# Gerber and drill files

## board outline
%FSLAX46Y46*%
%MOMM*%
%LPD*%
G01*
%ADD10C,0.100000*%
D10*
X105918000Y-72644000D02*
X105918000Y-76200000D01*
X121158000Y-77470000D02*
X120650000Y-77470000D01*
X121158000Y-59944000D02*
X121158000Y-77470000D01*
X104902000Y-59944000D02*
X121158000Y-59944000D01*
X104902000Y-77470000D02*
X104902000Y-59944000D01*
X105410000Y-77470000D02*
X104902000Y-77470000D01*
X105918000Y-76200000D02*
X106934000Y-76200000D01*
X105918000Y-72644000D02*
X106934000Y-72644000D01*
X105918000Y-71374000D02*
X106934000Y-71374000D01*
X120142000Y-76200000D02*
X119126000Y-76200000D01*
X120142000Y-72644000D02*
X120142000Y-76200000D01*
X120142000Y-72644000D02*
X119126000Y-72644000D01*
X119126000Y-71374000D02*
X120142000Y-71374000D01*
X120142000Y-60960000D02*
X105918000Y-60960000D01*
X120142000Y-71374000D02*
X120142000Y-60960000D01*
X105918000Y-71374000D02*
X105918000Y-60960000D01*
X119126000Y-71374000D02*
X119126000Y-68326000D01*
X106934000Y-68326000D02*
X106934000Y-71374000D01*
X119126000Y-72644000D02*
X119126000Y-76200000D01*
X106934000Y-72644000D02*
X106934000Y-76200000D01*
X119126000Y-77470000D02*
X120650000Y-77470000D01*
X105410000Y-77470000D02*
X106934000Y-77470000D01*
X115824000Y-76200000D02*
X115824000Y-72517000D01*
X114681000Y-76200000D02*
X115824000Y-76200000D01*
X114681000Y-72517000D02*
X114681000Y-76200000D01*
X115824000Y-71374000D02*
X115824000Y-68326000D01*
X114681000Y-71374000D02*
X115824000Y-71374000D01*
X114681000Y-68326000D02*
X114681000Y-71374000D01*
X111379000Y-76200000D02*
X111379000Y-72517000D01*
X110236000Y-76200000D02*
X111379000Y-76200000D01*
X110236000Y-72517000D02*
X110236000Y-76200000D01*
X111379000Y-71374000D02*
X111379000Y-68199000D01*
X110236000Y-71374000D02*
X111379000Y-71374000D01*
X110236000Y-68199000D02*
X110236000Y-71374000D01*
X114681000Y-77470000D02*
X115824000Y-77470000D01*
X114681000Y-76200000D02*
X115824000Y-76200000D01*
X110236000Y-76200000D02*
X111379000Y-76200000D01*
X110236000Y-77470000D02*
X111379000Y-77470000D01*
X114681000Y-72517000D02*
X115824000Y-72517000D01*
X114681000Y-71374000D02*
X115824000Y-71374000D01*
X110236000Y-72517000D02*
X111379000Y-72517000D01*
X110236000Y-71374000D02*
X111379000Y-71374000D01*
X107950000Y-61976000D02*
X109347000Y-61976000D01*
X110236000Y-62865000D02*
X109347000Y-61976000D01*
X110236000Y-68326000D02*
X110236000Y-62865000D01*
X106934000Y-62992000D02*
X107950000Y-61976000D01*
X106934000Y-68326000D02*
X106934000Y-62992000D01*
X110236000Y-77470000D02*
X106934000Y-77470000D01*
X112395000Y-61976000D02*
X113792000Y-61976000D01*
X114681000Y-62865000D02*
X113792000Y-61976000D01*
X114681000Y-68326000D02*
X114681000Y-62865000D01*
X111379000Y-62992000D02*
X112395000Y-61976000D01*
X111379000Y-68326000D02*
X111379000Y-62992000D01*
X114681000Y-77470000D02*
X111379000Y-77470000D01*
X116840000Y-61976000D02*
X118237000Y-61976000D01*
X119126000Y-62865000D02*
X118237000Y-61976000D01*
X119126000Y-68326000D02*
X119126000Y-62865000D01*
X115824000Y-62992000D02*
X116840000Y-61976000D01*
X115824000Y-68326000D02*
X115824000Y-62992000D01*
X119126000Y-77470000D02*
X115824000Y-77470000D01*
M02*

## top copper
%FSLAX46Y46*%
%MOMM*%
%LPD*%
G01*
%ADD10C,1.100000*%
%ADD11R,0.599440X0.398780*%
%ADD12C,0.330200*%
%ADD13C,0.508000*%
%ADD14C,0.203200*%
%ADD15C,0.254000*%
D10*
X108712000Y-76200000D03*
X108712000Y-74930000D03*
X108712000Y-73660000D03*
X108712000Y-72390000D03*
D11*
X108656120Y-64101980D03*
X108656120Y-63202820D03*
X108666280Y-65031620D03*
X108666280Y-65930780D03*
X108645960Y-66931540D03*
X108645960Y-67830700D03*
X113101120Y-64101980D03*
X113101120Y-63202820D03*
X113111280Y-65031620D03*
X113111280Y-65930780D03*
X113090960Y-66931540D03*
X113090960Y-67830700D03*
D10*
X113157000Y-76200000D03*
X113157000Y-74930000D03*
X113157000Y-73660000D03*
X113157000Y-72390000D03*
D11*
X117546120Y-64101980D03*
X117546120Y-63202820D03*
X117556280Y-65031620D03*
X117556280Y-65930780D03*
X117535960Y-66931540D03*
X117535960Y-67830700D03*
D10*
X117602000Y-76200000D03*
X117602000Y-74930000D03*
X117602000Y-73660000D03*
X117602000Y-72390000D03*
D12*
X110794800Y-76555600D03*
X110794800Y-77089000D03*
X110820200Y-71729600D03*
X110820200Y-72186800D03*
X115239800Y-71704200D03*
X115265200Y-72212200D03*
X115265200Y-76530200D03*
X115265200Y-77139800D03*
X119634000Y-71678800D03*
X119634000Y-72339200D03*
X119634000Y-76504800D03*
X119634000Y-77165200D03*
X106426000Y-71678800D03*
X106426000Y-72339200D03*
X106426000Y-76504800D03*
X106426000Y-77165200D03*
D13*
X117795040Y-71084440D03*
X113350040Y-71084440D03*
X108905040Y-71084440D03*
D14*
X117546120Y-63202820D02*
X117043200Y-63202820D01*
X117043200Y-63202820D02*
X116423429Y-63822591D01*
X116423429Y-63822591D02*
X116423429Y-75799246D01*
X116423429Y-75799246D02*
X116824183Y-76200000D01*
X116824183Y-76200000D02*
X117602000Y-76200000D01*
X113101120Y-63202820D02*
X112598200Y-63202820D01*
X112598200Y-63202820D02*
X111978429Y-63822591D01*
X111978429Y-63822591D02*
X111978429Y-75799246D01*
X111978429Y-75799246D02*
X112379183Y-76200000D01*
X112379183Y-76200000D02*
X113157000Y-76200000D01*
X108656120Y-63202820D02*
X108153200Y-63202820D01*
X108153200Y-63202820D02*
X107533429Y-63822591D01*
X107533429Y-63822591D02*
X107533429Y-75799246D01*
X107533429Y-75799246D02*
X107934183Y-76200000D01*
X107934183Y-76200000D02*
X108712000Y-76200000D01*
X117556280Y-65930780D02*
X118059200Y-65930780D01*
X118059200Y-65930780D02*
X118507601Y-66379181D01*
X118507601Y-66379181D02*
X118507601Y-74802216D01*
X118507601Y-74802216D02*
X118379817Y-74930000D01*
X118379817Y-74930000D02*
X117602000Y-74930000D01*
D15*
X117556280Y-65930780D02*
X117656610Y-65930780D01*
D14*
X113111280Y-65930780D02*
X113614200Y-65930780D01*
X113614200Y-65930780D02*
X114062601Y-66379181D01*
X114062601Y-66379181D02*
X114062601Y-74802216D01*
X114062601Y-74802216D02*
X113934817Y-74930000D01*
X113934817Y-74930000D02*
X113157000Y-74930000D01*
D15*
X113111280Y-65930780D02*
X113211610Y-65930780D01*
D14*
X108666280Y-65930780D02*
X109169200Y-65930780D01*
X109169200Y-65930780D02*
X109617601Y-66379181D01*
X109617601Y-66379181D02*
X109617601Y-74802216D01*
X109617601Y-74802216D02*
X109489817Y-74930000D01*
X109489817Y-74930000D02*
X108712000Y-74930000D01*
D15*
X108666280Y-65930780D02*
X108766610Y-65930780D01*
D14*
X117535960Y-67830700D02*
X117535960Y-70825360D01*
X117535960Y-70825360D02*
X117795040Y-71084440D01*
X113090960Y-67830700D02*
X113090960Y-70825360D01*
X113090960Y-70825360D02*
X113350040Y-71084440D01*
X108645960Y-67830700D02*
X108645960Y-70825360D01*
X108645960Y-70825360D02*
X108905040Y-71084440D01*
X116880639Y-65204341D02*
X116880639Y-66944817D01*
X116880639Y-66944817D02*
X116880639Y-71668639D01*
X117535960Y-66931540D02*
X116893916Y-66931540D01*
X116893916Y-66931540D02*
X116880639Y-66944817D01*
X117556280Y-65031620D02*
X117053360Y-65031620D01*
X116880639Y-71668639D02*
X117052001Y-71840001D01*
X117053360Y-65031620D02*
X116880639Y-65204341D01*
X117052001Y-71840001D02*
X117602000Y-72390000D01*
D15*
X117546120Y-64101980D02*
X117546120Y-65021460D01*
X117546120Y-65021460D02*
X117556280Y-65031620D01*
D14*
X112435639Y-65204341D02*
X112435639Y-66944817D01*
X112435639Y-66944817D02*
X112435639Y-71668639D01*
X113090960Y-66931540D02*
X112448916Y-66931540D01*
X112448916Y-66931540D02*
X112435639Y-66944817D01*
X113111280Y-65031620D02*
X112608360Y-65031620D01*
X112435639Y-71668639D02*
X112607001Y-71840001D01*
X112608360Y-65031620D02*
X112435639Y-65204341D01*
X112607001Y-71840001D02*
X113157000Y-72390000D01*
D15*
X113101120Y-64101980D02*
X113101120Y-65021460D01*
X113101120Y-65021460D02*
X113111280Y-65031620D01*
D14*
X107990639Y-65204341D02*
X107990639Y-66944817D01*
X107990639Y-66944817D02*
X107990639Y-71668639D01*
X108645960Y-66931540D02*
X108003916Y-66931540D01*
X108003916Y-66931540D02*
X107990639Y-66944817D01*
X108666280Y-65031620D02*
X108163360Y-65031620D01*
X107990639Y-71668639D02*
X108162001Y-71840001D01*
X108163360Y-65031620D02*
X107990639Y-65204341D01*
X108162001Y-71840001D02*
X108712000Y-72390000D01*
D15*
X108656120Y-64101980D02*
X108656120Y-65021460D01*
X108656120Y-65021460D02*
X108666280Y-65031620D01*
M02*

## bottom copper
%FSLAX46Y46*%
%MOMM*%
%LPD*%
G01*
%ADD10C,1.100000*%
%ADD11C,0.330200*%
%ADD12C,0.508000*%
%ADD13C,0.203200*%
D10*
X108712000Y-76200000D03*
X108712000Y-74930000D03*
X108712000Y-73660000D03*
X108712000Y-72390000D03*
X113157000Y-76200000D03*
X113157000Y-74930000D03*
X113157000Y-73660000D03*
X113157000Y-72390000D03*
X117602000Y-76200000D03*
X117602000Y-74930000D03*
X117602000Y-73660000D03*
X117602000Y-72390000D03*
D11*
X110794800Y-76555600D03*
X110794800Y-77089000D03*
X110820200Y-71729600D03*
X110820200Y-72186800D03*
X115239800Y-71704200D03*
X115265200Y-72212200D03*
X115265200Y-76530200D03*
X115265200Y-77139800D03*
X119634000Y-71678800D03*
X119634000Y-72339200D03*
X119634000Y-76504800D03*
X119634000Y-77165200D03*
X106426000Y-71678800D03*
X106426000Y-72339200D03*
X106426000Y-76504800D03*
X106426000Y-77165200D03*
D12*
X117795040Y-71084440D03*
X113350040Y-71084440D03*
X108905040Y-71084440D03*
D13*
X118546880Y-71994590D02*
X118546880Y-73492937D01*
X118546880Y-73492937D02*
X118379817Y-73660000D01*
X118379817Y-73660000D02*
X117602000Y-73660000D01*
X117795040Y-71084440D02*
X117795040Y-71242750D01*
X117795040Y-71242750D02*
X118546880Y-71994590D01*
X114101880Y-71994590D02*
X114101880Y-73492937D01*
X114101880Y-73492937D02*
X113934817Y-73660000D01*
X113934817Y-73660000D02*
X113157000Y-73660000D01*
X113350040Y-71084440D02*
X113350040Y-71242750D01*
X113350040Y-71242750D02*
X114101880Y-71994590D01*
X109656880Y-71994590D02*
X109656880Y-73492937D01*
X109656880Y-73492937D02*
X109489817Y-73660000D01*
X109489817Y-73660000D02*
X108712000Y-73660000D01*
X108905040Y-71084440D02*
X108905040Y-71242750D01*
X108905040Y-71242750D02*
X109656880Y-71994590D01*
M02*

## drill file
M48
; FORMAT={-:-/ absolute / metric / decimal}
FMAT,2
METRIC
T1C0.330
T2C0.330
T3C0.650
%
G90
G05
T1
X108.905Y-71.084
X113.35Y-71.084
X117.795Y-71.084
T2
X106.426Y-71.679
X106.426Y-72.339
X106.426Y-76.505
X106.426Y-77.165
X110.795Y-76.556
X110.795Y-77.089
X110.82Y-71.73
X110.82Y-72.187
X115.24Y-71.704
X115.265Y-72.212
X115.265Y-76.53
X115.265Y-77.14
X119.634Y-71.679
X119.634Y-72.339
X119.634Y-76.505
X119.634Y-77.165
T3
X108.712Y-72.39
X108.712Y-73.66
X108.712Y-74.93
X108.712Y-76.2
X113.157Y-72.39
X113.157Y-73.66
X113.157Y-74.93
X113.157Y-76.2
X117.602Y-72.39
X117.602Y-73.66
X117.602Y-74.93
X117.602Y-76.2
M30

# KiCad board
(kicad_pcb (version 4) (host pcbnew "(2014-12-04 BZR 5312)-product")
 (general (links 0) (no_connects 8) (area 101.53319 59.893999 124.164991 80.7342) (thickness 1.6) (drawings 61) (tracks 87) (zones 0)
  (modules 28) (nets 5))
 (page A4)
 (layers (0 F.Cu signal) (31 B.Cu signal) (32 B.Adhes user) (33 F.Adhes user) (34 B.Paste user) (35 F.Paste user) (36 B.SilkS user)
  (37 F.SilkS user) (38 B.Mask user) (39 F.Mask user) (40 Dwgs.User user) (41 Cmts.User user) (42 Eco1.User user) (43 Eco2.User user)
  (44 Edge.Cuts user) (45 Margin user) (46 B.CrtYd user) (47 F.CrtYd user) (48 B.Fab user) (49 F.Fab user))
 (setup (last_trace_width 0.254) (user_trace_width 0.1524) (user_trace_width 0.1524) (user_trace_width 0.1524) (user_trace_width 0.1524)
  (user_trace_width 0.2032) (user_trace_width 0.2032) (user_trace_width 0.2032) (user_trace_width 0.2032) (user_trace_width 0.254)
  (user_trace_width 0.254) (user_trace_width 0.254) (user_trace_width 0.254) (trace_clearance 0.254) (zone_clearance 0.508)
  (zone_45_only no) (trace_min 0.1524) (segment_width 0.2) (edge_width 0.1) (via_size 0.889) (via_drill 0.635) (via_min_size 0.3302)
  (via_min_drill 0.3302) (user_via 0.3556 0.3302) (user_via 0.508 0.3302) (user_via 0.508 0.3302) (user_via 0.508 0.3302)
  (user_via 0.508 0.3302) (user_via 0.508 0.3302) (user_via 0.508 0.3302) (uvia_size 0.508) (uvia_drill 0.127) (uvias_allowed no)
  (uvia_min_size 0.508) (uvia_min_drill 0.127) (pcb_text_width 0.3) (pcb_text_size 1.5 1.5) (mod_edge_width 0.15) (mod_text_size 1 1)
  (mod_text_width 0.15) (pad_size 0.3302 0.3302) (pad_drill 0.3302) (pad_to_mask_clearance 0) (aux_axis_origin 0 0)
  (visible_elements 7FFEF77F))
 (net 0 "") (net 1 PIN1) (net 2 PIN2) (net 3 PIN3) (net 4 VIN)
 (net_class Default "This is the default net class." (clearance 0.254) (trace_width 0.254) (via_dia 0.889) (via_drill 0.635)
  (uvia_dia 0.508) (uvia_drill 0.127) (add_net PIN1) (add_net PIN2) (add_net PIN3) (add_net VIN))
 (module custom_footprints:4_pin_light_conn (layer F.Cu) (at 112.522 76.2 90)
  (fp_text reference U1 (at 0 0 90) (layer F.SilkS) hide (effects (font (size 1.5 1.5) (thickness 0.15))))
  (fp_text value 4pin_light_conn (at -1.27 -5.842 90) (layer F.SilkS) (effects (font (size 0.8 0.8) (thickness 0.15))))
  (pad 1 thru_hole circle (at 0 -3.81 90) (size 1.1 1.1) (drill 0.65) (layers *.Cu *.Mask F.SilkS) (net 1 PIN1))
  (pad 2 thru_hole circle (at 1.27 -3.81 90) (size 1.1 1.1) (drill 0.65) (layers *.Cu *.Mask F.SilkS) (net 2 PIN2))
  (pad 3 thru_hole circle (at 2.54 -3.81 90) (size 1.1 1.1) (drill 0.65) (layers *.Cu *.Mask F.SilkS) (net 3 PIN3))
  (pad 4 thru_hole circle (at 3.81 -3.81 90) (size 1.1 1.1) (drill 0.65) (layers *.Cu *.Mask F.SilkS) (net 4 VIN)))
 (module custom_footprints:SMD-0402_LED (layer F.Cu) (at 108.65612 63.6524 90)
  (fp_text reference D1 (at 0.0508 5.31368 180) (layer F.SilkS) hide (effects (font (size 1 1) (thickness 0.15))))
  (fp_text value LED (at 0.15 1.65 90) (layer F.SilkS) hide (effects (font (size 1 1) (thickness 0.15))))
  (pad 1 smd rect (at -0.44958 0 90) (size 0.39878 0.59944) (layers F.Cu F.Paste F.Mask) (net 4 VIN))
  (pad 2 smd rect (at 0.44958 0 90) (size 0.39878 0.59944) (layers F.Cu F.Paste F.Mask) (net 1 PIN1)))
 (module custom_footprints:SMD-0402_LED (layer F.Cu) (at 108.66628 65.4812 270)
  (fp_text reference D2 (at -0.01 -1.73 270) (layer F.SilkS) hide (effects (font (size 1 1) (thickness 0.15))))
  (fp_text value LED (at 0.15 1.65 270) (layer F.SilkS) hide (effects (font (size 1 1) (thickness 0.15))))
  (pad 1 smd rect (at -0.44958 0 270) (size 0.39878 0.59944) (layers F.Cu F.Paste F.Mask) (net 4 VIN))
  (pad 2 smd rect (at 0.44958 0 270) (size 0.39878 0.59944) (layers F.Cu F.Paste F.Mask) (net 2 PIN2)))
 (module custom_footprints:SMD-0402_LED (layer F.Cu) (at 108.64596 67.38112 270)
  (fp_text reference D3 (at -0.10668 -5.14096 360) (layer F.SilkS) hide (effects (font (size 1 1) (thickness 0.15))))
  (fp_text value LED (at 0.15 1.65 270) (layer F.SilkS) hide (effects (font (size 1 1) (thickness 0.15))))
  (pad 1 smd rect (at -0.44958 0 270) (size 0.39878 0.59944) (layers F.Cu F.Paste F.Mask) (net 4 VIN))
  (pad 2 smd rect (at 0.44958 0 270) (size 0.39878 0.59944) (layers F.Cu F.Paste F.Mask) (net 3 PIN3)))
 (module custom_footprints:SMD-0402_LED (layer F.Cu) (at 113.10112 63.6524 90)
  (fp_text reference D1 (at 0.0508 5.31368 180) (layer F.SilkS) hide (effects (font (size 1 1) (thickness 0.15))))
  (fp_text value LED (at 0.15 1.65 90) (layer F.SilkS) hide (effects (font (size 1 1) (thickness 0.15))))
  (pad 1 smd rect (at -0.44958 0 90) (size 0.39878 0.59944) (layers F.Cu F.Paste F.Mask) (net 4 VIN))
  (pad 2 smd rect (at 0.44958 0 90) (size 0.39878 0.59944) (layers F.Cu F.Paste F.Mask) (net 1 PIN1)))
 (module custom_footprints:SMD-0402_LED (layer F.Cu) (at 113.11128 65.4812 270)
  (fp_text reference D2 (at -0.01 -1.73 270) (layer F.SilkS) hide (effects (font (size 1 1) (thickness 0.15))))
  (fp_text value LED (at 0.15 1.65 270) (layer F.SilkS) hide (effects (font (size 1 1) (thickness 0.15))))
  (pad 1 smd rect (at -0.44958 0 270) (size 0.39878 0.59944) (layers F.Cu F.Paste F.Mask) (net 4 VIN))
  (pad 2 smd rect (at 0.44958 0 270) (size 0.39878 0.59944) (layers F.Cu F.Paste F.Mask) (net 2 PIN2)))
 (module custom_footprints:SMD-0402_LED (layer F.Cu) (at 113.09096 67.38112 270)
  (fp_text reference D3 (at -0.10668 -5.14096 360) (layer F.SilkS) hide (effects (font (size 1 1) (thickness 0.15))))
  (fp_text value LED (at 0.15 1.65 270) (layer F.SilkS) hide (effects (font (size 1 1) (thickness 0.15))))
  (pad 1 smd rect (at -0.44958 0 270) (size 0.39878 0.59944) (layers F.Cu F.Paste F.Mask) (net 4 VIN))
  (pad 2 smd rect (at 0.44958 0 270) (size 0.39878 0.59944) (layers F.Cu F.Paste F.Mask) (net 3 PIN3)))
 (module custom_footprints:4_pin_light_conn (layer F.Cu) (at 116.967 76.2 90)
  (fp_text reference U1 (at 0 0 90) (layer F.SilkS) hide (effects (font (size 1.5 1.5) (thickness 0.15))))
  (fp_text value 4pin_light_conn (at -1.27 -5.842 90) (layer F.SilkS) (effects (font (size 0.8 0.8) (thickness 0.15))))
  (pad 1 thru_hole circle (at 0 -3.81 90) (size 1.1 1.1) (drill 0.65) (layers *.Cu *.Mask F.SilkS) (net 1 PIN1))
  (pad 2 thru_hole circle (at 1.27 -3.81 90) (size 1.1 1.1) (drill 0.65) (layers *.Cu *.Mask F.SilkS) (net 2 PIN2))
  (pad 3 thru_hole circle (at 2.54 -3.81 90) (size 1.1 1.1) (drill 0.65) (layers *.Cu *.Mask F.SilkS) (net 3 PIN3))
  (pad 4 thru_hole circle (at 3.81 -3.81 90) (size 1.1 1.1) (drill 0.65) (layers *.Cu *.Mask F.SilkS) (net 4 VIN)))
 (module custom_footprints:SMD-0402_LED (layer F.Cu) (at 117.54612 63.6524 90)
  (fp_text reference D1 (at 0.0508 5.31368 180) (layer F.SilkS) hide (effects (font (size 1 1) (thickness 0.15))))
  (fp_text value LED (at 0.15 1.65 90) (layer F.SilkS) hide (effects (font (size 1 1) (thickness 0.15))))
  (pad 1 smd rect (at -0.44958 0 90) (size 0.39878 0.59944) (layers F.Cu F.Paste F.Mask) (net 4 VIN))
  (pad 2 smd rect (at 0.44958 0 90) (size 0.39878 0.59944) (layers F.Cu F.Paste F.Mask) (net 1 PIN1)))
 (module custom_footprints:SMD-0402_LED (layer F.Cu) (at 117.55628 65.4812 270)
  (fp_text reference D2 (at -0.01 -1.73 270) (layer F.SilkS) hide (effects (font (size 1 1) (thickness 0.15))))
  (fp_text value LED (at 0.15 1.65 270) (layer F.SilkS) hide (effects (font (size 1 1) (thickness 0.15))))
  (pad 1 smd rect (at -0.44958 0 270) (size 0.39878 0.59944) (layers F.Cu F.Paste F.Mask) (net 4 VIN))
  (pad 2 smd rect (at 0.44958 0 270) (size 0.39878 0.59944) (layers F.Cu F.Paste F.Mask) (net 2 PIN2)))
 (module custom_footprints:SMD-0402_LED (layer F.Cu) (at 117.53596 67.38112 270)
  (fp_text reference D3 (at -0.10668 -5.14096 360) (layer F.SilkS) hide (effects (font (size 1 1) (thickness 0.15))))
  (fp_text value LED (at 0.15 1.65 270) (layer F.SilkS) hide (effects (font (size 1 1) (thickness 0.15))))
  (pad 1 smd rect (at -0.44958 0 270) (size 0.39878 0.59944) (layers F.Cu F.Paste F.Mask) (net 4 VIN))
  (pad 2 smd rect (at 0.44958 0 270) (size 0.39878 0.59944) (layers F.Cu F.Paste F.Mask) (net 3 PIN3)))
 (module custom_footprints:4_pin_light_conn (layer F.Cu) (at 121.412 76.2 90)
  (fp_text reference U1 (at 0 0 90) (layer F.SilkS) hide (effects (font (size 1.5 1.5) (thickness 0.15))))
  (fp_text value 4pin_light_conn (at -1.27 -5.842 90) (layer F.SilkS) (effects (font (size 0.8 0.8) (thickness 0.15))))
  (pad 1 thru_hole circle (at 0 -3.81 90) (size 1.1 1.1) (drill 0.65) (layers *.Cu *.Mask F.SilkS) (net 1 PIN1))
  (pad 2 thru_hole circle (at 1.27 -3.81 90) (size 1.1 1.1) (drill 0.65) (layers *.Cu *.Mask F.SilkS) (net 2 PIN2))
  (pad 3 thru_hole circle (at 2.54 -3.81 90) (size 1.1 1.1) (drill 0.65) (layers *.Cu *.Mask F.SilkS) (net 3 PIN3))
  (pad 4 thru_hole circle (at 3.81 -3.81 90) (size 1.1 1.1) (drill 0.65) (layers *.Cu *.Mask F.SilkS) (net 4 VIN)))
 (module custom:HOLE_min (layer F.Cu) (at 110.7948 76.5556)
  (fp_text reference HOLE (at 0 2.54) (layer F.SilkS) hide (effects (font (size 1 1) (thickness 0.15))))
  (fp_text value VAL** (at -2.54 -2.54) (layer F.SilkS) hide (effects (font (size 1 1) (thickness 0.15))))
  (pad 1 thru_hole circle (at 0 0) (size 0.3302 0.3302) (drill 0.3302) (layers *.Cu *.Mask F.SilkS)))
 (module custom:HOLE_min (layer F.Cu) (at 110.7948 77.089)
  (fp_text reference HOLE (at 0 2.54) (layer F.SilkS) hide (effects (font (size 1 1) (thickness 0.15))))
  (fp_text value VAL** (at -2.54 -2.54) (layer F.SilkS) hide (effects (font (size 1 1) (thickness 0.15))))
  (pad 1 thru_hole circle (at 0 0) (size 0.3302 0.3302) (drill 0.3302) (layers *.Cu *.Mask F.SilkS)))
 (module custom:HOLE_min (layer F.Cu) (at 110.8202 71.7296)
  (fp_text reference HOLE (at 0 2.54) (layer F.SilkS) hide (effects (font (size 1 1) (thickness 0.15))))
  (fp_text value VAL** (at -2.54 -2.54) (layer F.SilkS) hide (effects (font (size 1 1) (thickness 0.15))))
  (pad 1 thru_hole circle (at 0 0) (size 0.3302 0.3302) (drill 0.3302) (layers *.Cu *.Mask F.SilkS)))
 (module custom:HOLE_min (layer F.Cu) (at 110.8202 72.1868)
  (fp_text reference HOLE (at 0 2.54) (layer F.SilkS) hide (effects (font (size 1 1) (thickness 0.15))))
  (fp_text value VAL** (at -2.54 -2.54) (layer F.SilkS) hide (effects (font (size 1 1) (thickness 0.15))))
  (pad 1 thru_hole circle (at 0 0) (size 0.3302 0.3302) (drill 0.3302) (layers *.Cu *.Mask F.SilkS)))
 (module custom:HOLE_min (layer F.Cu) (at 115.2398 71.7042)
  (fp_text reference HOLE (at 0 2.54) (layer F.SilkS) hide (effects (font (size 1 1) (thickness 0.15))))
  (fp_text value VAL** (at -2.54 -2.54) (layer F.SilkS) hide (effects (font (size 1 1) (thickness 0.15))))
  (pad 1 thru_hole circle (at 0 0) (size 0.3302 0.3302) (drill 0.3302) (layers *.Cu *.Mask F.SilkS)))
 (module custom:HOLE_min (layer F.Cu) (at 115.2652 72.2122)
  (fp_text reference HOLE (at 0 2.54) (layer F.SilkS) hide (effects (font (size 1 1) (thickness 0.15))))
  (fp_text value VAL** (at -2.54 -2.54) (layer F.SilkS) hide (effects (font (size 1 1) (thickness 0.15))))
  (pad 1 thru_hole circle (at 0 0) (size 0.3302 0.3302) (drill 0.3302) (layers *.Cu *.Mask F.SilkS)))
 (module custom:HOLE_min (layer F.Cu) (at 115.2652 76.5302)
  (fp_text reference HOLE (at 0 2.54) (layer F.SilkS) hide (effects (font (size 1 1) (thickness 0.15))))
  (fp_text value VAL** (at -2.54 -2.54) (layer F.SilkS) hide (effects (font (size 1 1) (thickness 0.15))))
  (pad 1 thru_hole circle (at 0 0) (size 0.3302 0.3302) (drill 0.3302) (layers *.Cu *.Mask F.SilkS)))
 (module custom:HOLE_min (layer F.Cu) (at 115.2652 77.1398)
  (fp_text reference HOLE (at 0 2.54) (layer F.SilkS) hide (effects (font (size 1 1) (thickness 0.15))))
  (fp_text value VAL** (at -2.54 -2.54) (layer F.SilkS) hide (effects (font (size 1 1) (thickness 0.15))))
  (pad 1 thru_hole circle (at 0 0) (size 0.3302 0.3302) (drill 0.3302) (layers *.Cu *.Mask F.SilkS)))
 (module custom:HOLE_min (layer F.Cu) (at 119.634 71.6788)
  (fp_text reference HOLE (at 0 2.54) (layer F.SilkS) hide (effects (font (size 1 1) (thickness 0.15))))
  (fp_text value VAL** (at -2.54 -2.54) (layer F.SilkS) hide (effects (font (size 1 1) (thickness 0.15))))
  (pad 1 thru_hole circle (at 0 0) (size 0.3302 0.3302) (drill 0.3302) (layers *.Cu *.Mask F.SilkS)))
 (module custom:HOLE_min (layer F.Cu) (at 119.634 72.3392)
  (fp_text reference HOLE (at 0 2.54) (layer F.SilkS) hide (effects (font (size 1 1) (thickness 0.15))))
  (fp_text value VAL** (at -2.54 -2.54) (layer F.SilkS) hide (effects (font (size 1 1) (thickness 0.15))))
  (pad 1 thru_hole circle (at 0 0) (size 0.3302 0.3302) (drill 0.3302) (layers *.Cu *.Mask F.SilkS)))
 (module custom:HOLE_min (layer F.Cu) (at 119.634 76.5048)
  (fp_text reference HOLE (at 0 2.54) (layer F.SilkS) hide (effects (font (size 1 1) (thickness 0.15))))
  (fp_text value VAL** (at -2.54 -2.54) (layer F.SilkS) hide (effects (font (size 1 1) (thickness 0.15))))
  (pad 1 thru_hole circle (at 0 0) (size 0.3302 0.3302) (drill 0.3302) (layers *.Cu *.Mask F.SilkS)))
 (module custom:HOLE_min (layer F.Cu) (at 119.634 77.1652)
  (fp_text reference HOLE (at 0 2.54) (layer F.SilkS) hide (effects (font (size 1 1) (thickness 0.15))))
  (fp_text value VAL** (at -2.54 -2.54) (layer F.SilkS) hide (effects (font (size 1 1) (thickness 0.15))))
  (pad 1 thru_hole circle (at 0 0) (size 0.3302 0.3302) (drill 0.3302) (layers *.Cu *.Mask F.SilkS)))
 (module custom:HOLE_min (layer F.Cu) (at 106.426 71.6788)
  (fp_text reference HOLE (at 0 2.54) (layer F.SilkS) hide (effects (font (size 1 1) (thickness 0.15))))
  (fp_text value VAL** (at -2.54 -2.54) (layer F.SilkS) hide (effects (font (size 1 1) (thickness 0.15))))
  (pad 1 thru_hole circle (at 0 0) (size 0.3302 0.3302) (drill 0.3302) (layers *.Cu *.Mask F.SilkS)))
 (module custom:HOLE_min (layer F.Cu) (at 106.426 72.3392)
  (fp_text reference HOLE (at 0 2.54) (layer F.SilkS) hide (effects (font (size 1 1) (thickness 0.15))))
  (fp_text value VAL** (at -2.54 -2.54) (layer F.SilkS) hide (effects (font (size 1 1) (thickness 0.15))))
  (pad 1 thru_hole circle (at 0 0) (size 0.3302 0.3302) (drill 0.3302) (layers *.Cu *.Mask F.SilkS)))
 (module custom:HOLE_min (layer F.Cu) (at 106.426 76.5048)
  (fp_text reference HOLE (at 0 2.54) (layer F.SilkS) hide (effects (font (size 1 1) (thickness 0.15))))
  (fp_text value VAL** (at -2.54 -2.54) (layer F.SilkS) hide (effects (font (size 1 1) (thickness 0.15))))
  (pad 1 thru_hole circle (at 0 0) (size 0.3302 0.3302) (drill 0.3302) (layers *.Cu *.Mask F.SilkS)))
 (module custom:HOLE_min (layer F.Cu) (at 106.426 77.1652)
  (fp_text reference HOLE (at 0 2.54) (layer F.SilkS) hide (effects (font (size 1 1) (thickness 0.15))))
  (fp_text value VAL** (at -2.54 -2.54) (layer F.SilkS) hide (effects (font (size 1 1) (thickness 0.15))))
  (pad 1 thru_hole circle (at 0 0) (size 0.3302 0.3302) (drill 0.3302) (layers *.Cu *.Mask F.SilkS)))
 (gr_line (start 105.918 72.644) (end 105.918 76.2) (angle 90) (layer Edge.Cuts) (width 0.1))
 (gr_line (start 121.158 77.47) (end 120.65 77.47) (angle 90) (layer Edge.Cuts) (width 0.1))
 (gr_line (start 121.158 59.944) (end 121.158 77.47) (angle 90) (layer Edge.Cuts) (width 0.1))
 (gr_line (start 104.902 59.944) (end 121.158 59.944) (angle 90) (layer Edge.Cuts) (width 0.1))
 (gr_line (start 104.902 77.47) (end 104.902 59.944) (angle 90) (layer Edge.Cuts) (width 0.1))
 (gr_line (start 105.41 77.47) (end 104.902 77.47) (angle 90) (layer Edge.Cuts) (width 0.1))
 (gr_line (start 105.918 76.2) (end 106.934 76.2) (angle 90) (layer Edge.Cuts) (width 0.1))
 (gr_line (start 105.918 72.644) (end 106.934 72.644) (angle 90) (layer Edge.Cuts) (width 0.1))
 (gr_line (start 105.918 71.374) (end 106.934 71.374) (angle 90) (layer Edge.Cuts) (width 0.1))
 (gr_line (start 120.142 76.2) (end 119.126 76.2) (angle 90) (layer Edge.Cuts) (width 0.1))
 (gr_line (start 120.142 72.644) (end 120.142 76.2) (angle 90) (layer Edge.Cuts) (width 0.1))
 (gr_line (start 120.142 72.644) (end 119.126 72.644) (angle 90) (layer Edge.Cuts) (width 0.1))
 (gr_line (start 119.126 71.374) (end 120.142 71.374) (angle 90) (layer Edge.Cuts) (width 0.1))
 (gr_line (start 120.142 60.96) (end 105.918 60.96) (angle 90) (layer Edge.Cuts) (width 0.1))
 (gr_line (start 120.142 71.374) (end 120.142 60.96) (angle 90) (layer Edge.Cuts) (width 0.1))
 (gr_line (start 105.918 71.374) (end 105.918 60.96) (angle 90) (layer Edge.Cuts) (width 0.1))
 (gr_line (start 119.126 71.374) (end 119.126 68.326) (angle 90) (layer Edge.Cuts) (width 0.1))
 (gr_line (start 106.934 68.326) (end 106.934 71.374) (angle 90) (layer Edge.Cuts) (width 0.1))
 (gr_line (start 119.126 72.644) (end 119.126 76.2) (angle 90) (layer Edge.Cuts) (width 0.1))
 (gr_line (start 106.934 72.644) (end 106.934 76.2) (angle 90) (layer Edge.Cuts) (width 0.1))
 (gr_line (start 119.126 77.47) (end 120.65 77.47) (angle 90) (layer Edge.Cuts) (width 0.1))
 (gr_line (start 105.41 77.47) (end 106.934 77.47) (angle 90) (layer Edge.Cuts) (width 0.1))
 (gr_line (start 115.824 76.2) (end 115.824 72.517) (angle 90) (layer Edge.Cuts) (width 0.1))
 (gr_line (start 114.681 76.2) (end 115.824 76.2) (angle 90) (layer Edge.Cuts) (width 0.1))
 (gr_line (start 114.681 72.517) (end 114.681 76.2) (angle 90) (layer Edge.Cuts) (width 0.1))
 (gr_line (start 115.824 71.374) (end 115.824 68.326) (angle 90) (layer Edge.Cuts) (width 0.1))
 (gr_line (start 114.681 71.374) (end 115.824 71.374) (angle 90) (layer Edge.Cuts) (width 0.1))
 (gr_line (start 114.681 68.326) (end 114.681 71.374) (angle 90) (layer Edge.Cuts) (width 0.1))
 (gr_line (start 111.379 76.2) (end 111.379 72.517) (angle 90) (layer Edge.Cuts) (width 0.1))
 (gr_line (start 110.236 76.2) (end 111.379 76.2) (angle 90) (layer Edge.Cuts) (width 0.1))
 (gr_line (start 110.236 72.517) (end 110.236 76.2) (angle 90) (layer Edge.Cuts) (width 0.1))
 (gr_line (start 111.379 71.374) (end 111.379 68.199) (angle 90) (layer Edge.Cuts) (width 0.1))
 (gr_line (start 110.236 71.374) (end 111.379 71.374) (angle 90) (layer Edge.Cuts) (width 0.1))
 (gr_line (start 110.236 68.199) (end 110.236 71.374) (angle 90) (layer Edge.Cuts) (width 0.1))
 (gr_line (start 114.681 77.47) (end 115.824 77.47) (angle 90) (layer Edge.Cuts) (width 0.1))
 (gr_line (start 114.681 76.2) (end 115.824 76.2) (angle 90) (layer Edge.Cuts) (width 0.1))
 (gr_line (start 110.236 76.2) (end 111.379 76.2) (angle 90) (layer Edge.Cuts) (width 0.1))
 (gr_line (start 110.236 77.47) (end 111.379 77.47) (angle 90) (layer Edge.Cuts) (width 0.1))
 (gr_line (start 114.681 72.517) (end 115.824 72.517) (angle 90) (layer Edge.Cuts) (width 0.1))
 (gr_line (start 114.681 71.374) (end 115.824 71.374) (angle 90) (layer Edge.Cuts) (width 0.1))
 (gr_line (start 110.236 72.517) (end 111.379 72.517) (angle 90) (layer Edge.Cuts) (width 0.1))
 (gr_line (start 110.236 71.374) (end 111.379 71.374) (angle 90) (layer Edge.Cuts) (width 0.1))
 (gr_line (start 107.95 61.976) (end 109.347 61.976) (angle 90) (layer Edge.Cuts) (width 0.1))
 (gr_line (start 110.236 62.865) (end 109.347 61.976) (angle 90) (layer Edge.Cuts) (width 0.1))
 (gr_line (start 110.236 68.326) (end 110.236 62.865) (angle 90) (layer Edge.Cuts) (width 0.1))
 (gr_line (start 106.934 62.992) (end 107.95 61.976) (angle 90) (layer Edge.Cuts) (width 0.1))
 (gr_line (start 106.934 68.326) (end 106.934 62.992) (angle 90) (layer Edge.Cuts) (width 0.1))
 (gr_line (start 110.236 77.47) (end 106.934 77.47) (angle 90) (layer Edge.Cuts) (width 0.1))
 (gr_line (start 112.395 61.976) (end 113.792 61.976) (angle 90) (layer Edge.Cuts) (width 0.1))
 (gr_line (start 114.681 62.865) (end 113.792 61.976) (angle 90) (layer Edge.Cuts) (width 0.1))
 (gr_line (start 114.681 68.326) (end 114.681 62.865) (angle 90) (layer Edge.Cuts) (width 0.1))
 (gr_line (start 111.379 62.992) (end 112.395 61.976) (angle 90) (layer Edge.Cuts) (width 0.1))
 (gr_line (start 111.379 68.326) (end 111.379 62.992) (angle 90) (layer Edge.Cuts) (width 0.1))
 (gr_line (start 114.681 77.47) (end 111.379 77.47) (angle 90) (layer Edge.Cuts) (width 0.1))
 (gr_line (start 116.84 61.976) (end 118.237 61.976) (angle 90) (layer Edge.Cuts) (width 0.1))
 (gr_line (start 119.126 62.865) (end 118.237 61.976) (angle 90) (layer Edge.Cuts) (width 0.1))
 (gr_line (start 119.126 68.326) (end 119.126 62.865) (angle 90) (layer Edge.Cuts) (width 0.1))
 (gr_line (start 115.824 62.992) (end 116.84 61.976) (angle 90) (layer Edge.Cuts) (width 0.1))
 (gr_line (start 115.824 68.326) (end 115.824 62.992) (angle 90) (layer Edge.Cuts) (width 0.1))
 (gr_line (start 119.126 77.47) (end 115.824 77.47) (angle 90) (layer Edge.Cuts) (width 0.1))
 (segment (start 117.54612 63.20282) (end 117.0432 63.20282) (width 0.2032) (layer F.Cu) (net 1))
 (segment (start 117.0432 63.20282) (end 116.423429 63.822591) (width 0.2032) (layer F.Cu) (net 1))
 (segment (start 116.423429 63.822591) (end 116.423429 75.799246) (width 0.2032) (layer F.Cu) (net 1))
 (segment (start 116.423429 75.799246) (end 116.824183 76.2) (width 0.2032) (layer F.Cu) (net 1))
 (segment (start 116.824183 76.2) (end 117.602 76.2) (width 0.2032) (layer F.Cu) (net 1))
 (segment (start 113.10112 63.20282) (end 112.5982 63.20282) (width 0.2032) (layer F.Cu) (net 1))
 (segment (start 112.5982 63.20282) (end 111.978429 63.822591) (width 0.2032) (layer F.Cu) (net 1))
 (segment (start 111.978429 63.822591) (end 111.978429 75.799246) (width 0.2032) (layer F.Cu) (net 1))
 (segment (start 111.978429 75.799246) (end 112.379183 76.2) (width 0.2032) (layer F.Cu) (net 1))
 (segment (start 112.379183 76.2) (end 113.157 76.2) (width 0.2032) (layer F.Cu) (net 1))
 (segment (start 108.65612 63.20282) (end 108.1532 63.20282) (width 0.2032) (layer F.Cu) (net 1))
 (segment (start 108.1532 63.20282) (end 107.533429 63.822591) (width 0.2032) (layer F.Cu) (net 1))
 (segment (start 107.533429 63.822591) (end 107.533429 75.799246) (width 0.2032) (layer F.Cu) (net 1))
 (segment (start 107.533429 75.799246) (end 107.934183 76.2) (width 0.2032) (layer F.Cu) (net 1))
 (segment (start 107.934183 76.2) (end 108.712 76.2) (width 0.2032) (layer F.Cu) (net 1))
 (segment (start 117.55628 65.93078) (end 118.0592 65.93078) (width 0.2032) (layer F.Cu) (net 2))
 (segment (start 118.0592 65.93078) (end 118.507601 66.379181) (width 0.2032) (layer F.Cu) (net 2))
 (segment (start 118.507601 66.379181) (end 118.507601 74.802216) (width 0.2032) (layer F.Cu) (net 2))
 (segment (start 118.507601 74.802216) (end 118.379817 74.93) (width 0.2032) (layer F.Cu) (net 2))
 (segment (start 118.379817 74.93) (end 117.602 74.93) (width 0.2032) (layer F.Cu) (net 2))
 (segment (start 117.55628 65.93078) (end 117.65661 65.93078) (width 0.254) (layer F.Cu) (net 2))
 (segment (start 113.11128 65.93078) (end 113.6142 65.93078) (width 0.2032) (layer F.Cu) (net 2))
 (segment (start 113.6142 65.93078) (end 114.062601 66.379181) (width 0.2032) (layer F.Cu) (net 2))
 (segment (start 114.062601 66.379181) (end 114.062601 74.802216) (width 0.2032) (layer F.Cu) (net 2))
 (segment (start 114.062601 74.802216) (end 113.934817 74.93) (width 0.2032) (layer F.Cu) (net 2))
 (segment (start 113.934817 74.93) (end 113.157 74.93) (width 0.2032) (layer F.Cu) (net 2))
 (segment (start 113.11128 65.93078) (end 113.21161 65.93078) (width 0.254) (layer F.Cu) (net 2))
 (segment (start 108.66628 65.93078) (end 109.1692 65.93078) (width 0.2032) (layer F.Cu) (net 2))
 (segment (start 109.1692 65.93078) (end 109.617601 66.379181) (width 0.2032) (layer F.Cu) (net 2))
 (segment (start 109.617601 66.379181) (end 109.617601 74.802216) (width 0.2032) (layer F.Cu) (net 2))
 (segment (start 109.617601 74.802216) (end 109.489817 74.93) (width 0.2032) (layer F.Cu) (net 2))
 (segment (start 109.489817 74.93) (end 108.712 74.93) (width 0.2032) (layer F.Cu) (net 2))
 (segment (start 108.66628 65.93078) (end 108.76661 65.93078) (width 0.254) (layer F.Cu) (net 2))
 (segment (start 118.54688 71.99459) (end 118.54688 73.492937) (width 0.2032) (layer B.Cu) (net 3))
 (segment (start 118.54688 73.492937) (end 118.379817 73.66) (width 0.2032) (layer B.Cu) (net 3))
 (segment (start 118.379817 73.66) (end 117.602 73.66) (width 0.2032) (layer B.Cu) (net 3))
 (segment (start 117.79504 71.08444) (end 117.79504 71.24275) (width 0.2032) (layer B.Cu) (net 3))
 (segment (start 117.79504 71.24275) (end 118.54688 71.99459) (width 0.2032) (layer B.Cu) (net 3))
 (segment (start 117.53596 67.8307) (end 117.53596 70.82536) (width 0.2032) (layer F.Cu) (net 3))
 (segment (start 117.53596 70.82536) (end 117.79504 71.08444) (width 0.2032) (layer F.Cu) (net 3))
 (via (at 117.79504 71.08444) (size 0.508) (drill 0.3302) (layers F.Cu B.Cu) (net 3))
 (segment (start 114.10188 71.99459) (end 114.10188 73.492937) (width 0.2032) (layer B.Cu) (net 3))
 (segment (start 114.10188 73.492937) (end 113.934817 73.66) (width 0.2032) (layer B.Cu) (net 3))
 (segment (start 113.934817 73.66) (end 113.157 73.66) (width 0.2032) (layer B.Cu) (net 3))
 (segment (start 113.35004 71.08444) (end 113.35004 71.24275) (width 0.2032) (layer B.Cu) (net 3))
 (segment (start 113.35004 71.24275) (end 114.10188 71.99459) (width 0.2032) (layer B.Cu) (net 3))
 (segment (start 113.09096 67.8307) (end 113.09096 70.82536) (width 0.2032) (layer F.Cu) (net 3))
 (segment (start 113.09096 70.82536) (end 113.35004 71.08444) (width 0.2032) (layer F.Cu) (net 3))
 (via (at 113.35004 71.08444) (size 0.508) (drill 0.3302) (layers F.Cu B.Cu) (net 3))
 (segment (start 109.65688 71.99459) (end 109.65688 73.492937) (width 0.2032) (layer B.Cu) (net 3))
 (segment (start 109.65688 73.492937) (end 109.489817 73.66) (width 0.2032) (layer B.Cu) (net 3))
 (segment (start 109.489817 73.66) (end 108.712 73.66) (width 0.2032) (layer B.Cu) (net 3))
 (segment (start 108.90504 71.08444) (end 108.90504 71.24275) (width 0.2032) (layer B.Cu) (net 3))
 (segment (start 108.90504 71.24275) (end 109.65688 71.99459) (width 0.2032) (layer B.Cu) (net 3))
 (segment (start 108.64596 67.8307) (end 108.64596 70.82536) (width 0.2032) (layer F.Cu) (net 3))
 (segment (start 108.64596 70.82536) (end 108.90504 71.08444) (width 0.2032) (layer F.Cu) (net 3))
 (via (at 108.90504 71.08444) (size 0.508) (drill 0.3302) (layers F.Cu B.Cu) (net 3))
 (segment (start 116.880639 65.204341) (end 116.880639 66.944817) (width 0.2032) (layer F.Cu) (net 4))
 (segment (start 116.880639 66.944817) (end 116.880639 71.668639) (width 0.2032) (layer F.Cu) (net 4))
 (segment (start 117.53596 66.93154) (end 116.893916 66.93154) (width 0.2032) (layer F.Cu) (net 4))
 (segment (start 116.893916 66.93154) (end 116.880639 66.944817) (width 0.2032) (layer F.Cu) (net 4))
 (segment (start 117.55628 65.03162) (end 117.05336 65.03162) (width 0.2032) (layer F.Cu) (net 4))
 (segment (start 116.880639 71.668639) (end 117.052001 71.840001) (width 0.2032) (layer F.Cu) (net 4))
 (segment (start 117.05336 65.03162) (end 116.880639 65.204341) (width 0.2032) (layer F.Cu) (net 4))
 (segment (start 117.052001 71.840001) (end 117.602 72.39) (width 0.2032) (layer F.Cu) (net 4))
 (segment (start 117.54612 64.10198) (end 117.54612 65.02146) (width 0.254) (layer F.Cu) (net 4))
 (segment (start 117.54612 65.02146) (end 117.55628 65.03162) (width 0.254) (layer F.Cu) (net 4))
 (segment (start 112.435639 65.204341) (end 112.435639 66.944817) (width 0.2032) (layer F.Cu) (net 4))
 (segment (start 112.435639 66.944817) (end 112.435639 71.668639) (width 0.2032) (layer F.Cu) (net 4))
 (segment (start 113.09096 66.93154) (end 112.448916 66.93154) (width 0.2032) (layer F.Cu) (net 4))
 (segment (start 112.448916 66.93154) (end 112.435639 66.944817) (width 0.2032) (layer F.Cu) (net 4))
 (segment (start 113.11128 65.03162) (end 112.60836 65.03162) (width 0.2032) (layer F.Cu) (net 4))
 (segment (start 112.435639 71.668639) (end 112.607001 71.840001) (width 0.2032) (layer F.Cu) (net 4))
 (segment (start 112.60836 65.03162) (end 112.435639 65.204341) (width 0.2032) (layer F.Cu) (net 4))
 (segment (start 112.607001 71.840001) (end 113.157 72.39) (width 0.2032) (layer F.Cu) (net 4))
 (segment (start 113.10112 64.10198) (end 113.10112 65.02146) (width 0.254) (layer F.Cu) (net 4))
 (segment (start 113.10112 65.02146) (end 113.11128 65.03162) (width 0.254) (layer F.Cu) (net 4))
 (segment (start 107.990639 65.204341) (end 107.990639 66.944817) (width 0.2032) (layer F.Cu) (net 4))
 (segment (start 107.990639 66.944817) (end 107.990639 71.668639) (width 0.2032) (layer F.Cu) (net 4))
 (segment (start 108.64596 66.93154) (end 108.003916 66.93154) (width 0.2032) (layer F.Cu) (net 4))
 (segment (start 108.003916 66.93154) (end 107.990639 66.944817) (width 0.2032) (layer F.Cu) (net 4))
 (segment (start 108.66628 65.03162) (end 108.16336 65.03162) (width 0.2032) (layer F.Cu) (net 4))
 (segment (start 107.990639 71.668639) (end 108.162001 71.840001) (width 0.2032) (layer F.Cu) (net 4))
 (segment (start 108.16336 65.03162) (end 107.990639 65.204341) (width 0.2032) (layer F.Cu) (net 4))
 (segment (start 108.162001 71.840001) (end 108.712 72.39) (width 0.2032) (layer F.Cu) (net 4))
 (segment (start 108.65612 64.10198) (end 108.65612 65.02146) (width 0.254) (layer F.Cu) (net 4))
 (segment (start 108.65612 65.02146) (end 108.66628 65.03162) (width 0.254) (layer F.Cu) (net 4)))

